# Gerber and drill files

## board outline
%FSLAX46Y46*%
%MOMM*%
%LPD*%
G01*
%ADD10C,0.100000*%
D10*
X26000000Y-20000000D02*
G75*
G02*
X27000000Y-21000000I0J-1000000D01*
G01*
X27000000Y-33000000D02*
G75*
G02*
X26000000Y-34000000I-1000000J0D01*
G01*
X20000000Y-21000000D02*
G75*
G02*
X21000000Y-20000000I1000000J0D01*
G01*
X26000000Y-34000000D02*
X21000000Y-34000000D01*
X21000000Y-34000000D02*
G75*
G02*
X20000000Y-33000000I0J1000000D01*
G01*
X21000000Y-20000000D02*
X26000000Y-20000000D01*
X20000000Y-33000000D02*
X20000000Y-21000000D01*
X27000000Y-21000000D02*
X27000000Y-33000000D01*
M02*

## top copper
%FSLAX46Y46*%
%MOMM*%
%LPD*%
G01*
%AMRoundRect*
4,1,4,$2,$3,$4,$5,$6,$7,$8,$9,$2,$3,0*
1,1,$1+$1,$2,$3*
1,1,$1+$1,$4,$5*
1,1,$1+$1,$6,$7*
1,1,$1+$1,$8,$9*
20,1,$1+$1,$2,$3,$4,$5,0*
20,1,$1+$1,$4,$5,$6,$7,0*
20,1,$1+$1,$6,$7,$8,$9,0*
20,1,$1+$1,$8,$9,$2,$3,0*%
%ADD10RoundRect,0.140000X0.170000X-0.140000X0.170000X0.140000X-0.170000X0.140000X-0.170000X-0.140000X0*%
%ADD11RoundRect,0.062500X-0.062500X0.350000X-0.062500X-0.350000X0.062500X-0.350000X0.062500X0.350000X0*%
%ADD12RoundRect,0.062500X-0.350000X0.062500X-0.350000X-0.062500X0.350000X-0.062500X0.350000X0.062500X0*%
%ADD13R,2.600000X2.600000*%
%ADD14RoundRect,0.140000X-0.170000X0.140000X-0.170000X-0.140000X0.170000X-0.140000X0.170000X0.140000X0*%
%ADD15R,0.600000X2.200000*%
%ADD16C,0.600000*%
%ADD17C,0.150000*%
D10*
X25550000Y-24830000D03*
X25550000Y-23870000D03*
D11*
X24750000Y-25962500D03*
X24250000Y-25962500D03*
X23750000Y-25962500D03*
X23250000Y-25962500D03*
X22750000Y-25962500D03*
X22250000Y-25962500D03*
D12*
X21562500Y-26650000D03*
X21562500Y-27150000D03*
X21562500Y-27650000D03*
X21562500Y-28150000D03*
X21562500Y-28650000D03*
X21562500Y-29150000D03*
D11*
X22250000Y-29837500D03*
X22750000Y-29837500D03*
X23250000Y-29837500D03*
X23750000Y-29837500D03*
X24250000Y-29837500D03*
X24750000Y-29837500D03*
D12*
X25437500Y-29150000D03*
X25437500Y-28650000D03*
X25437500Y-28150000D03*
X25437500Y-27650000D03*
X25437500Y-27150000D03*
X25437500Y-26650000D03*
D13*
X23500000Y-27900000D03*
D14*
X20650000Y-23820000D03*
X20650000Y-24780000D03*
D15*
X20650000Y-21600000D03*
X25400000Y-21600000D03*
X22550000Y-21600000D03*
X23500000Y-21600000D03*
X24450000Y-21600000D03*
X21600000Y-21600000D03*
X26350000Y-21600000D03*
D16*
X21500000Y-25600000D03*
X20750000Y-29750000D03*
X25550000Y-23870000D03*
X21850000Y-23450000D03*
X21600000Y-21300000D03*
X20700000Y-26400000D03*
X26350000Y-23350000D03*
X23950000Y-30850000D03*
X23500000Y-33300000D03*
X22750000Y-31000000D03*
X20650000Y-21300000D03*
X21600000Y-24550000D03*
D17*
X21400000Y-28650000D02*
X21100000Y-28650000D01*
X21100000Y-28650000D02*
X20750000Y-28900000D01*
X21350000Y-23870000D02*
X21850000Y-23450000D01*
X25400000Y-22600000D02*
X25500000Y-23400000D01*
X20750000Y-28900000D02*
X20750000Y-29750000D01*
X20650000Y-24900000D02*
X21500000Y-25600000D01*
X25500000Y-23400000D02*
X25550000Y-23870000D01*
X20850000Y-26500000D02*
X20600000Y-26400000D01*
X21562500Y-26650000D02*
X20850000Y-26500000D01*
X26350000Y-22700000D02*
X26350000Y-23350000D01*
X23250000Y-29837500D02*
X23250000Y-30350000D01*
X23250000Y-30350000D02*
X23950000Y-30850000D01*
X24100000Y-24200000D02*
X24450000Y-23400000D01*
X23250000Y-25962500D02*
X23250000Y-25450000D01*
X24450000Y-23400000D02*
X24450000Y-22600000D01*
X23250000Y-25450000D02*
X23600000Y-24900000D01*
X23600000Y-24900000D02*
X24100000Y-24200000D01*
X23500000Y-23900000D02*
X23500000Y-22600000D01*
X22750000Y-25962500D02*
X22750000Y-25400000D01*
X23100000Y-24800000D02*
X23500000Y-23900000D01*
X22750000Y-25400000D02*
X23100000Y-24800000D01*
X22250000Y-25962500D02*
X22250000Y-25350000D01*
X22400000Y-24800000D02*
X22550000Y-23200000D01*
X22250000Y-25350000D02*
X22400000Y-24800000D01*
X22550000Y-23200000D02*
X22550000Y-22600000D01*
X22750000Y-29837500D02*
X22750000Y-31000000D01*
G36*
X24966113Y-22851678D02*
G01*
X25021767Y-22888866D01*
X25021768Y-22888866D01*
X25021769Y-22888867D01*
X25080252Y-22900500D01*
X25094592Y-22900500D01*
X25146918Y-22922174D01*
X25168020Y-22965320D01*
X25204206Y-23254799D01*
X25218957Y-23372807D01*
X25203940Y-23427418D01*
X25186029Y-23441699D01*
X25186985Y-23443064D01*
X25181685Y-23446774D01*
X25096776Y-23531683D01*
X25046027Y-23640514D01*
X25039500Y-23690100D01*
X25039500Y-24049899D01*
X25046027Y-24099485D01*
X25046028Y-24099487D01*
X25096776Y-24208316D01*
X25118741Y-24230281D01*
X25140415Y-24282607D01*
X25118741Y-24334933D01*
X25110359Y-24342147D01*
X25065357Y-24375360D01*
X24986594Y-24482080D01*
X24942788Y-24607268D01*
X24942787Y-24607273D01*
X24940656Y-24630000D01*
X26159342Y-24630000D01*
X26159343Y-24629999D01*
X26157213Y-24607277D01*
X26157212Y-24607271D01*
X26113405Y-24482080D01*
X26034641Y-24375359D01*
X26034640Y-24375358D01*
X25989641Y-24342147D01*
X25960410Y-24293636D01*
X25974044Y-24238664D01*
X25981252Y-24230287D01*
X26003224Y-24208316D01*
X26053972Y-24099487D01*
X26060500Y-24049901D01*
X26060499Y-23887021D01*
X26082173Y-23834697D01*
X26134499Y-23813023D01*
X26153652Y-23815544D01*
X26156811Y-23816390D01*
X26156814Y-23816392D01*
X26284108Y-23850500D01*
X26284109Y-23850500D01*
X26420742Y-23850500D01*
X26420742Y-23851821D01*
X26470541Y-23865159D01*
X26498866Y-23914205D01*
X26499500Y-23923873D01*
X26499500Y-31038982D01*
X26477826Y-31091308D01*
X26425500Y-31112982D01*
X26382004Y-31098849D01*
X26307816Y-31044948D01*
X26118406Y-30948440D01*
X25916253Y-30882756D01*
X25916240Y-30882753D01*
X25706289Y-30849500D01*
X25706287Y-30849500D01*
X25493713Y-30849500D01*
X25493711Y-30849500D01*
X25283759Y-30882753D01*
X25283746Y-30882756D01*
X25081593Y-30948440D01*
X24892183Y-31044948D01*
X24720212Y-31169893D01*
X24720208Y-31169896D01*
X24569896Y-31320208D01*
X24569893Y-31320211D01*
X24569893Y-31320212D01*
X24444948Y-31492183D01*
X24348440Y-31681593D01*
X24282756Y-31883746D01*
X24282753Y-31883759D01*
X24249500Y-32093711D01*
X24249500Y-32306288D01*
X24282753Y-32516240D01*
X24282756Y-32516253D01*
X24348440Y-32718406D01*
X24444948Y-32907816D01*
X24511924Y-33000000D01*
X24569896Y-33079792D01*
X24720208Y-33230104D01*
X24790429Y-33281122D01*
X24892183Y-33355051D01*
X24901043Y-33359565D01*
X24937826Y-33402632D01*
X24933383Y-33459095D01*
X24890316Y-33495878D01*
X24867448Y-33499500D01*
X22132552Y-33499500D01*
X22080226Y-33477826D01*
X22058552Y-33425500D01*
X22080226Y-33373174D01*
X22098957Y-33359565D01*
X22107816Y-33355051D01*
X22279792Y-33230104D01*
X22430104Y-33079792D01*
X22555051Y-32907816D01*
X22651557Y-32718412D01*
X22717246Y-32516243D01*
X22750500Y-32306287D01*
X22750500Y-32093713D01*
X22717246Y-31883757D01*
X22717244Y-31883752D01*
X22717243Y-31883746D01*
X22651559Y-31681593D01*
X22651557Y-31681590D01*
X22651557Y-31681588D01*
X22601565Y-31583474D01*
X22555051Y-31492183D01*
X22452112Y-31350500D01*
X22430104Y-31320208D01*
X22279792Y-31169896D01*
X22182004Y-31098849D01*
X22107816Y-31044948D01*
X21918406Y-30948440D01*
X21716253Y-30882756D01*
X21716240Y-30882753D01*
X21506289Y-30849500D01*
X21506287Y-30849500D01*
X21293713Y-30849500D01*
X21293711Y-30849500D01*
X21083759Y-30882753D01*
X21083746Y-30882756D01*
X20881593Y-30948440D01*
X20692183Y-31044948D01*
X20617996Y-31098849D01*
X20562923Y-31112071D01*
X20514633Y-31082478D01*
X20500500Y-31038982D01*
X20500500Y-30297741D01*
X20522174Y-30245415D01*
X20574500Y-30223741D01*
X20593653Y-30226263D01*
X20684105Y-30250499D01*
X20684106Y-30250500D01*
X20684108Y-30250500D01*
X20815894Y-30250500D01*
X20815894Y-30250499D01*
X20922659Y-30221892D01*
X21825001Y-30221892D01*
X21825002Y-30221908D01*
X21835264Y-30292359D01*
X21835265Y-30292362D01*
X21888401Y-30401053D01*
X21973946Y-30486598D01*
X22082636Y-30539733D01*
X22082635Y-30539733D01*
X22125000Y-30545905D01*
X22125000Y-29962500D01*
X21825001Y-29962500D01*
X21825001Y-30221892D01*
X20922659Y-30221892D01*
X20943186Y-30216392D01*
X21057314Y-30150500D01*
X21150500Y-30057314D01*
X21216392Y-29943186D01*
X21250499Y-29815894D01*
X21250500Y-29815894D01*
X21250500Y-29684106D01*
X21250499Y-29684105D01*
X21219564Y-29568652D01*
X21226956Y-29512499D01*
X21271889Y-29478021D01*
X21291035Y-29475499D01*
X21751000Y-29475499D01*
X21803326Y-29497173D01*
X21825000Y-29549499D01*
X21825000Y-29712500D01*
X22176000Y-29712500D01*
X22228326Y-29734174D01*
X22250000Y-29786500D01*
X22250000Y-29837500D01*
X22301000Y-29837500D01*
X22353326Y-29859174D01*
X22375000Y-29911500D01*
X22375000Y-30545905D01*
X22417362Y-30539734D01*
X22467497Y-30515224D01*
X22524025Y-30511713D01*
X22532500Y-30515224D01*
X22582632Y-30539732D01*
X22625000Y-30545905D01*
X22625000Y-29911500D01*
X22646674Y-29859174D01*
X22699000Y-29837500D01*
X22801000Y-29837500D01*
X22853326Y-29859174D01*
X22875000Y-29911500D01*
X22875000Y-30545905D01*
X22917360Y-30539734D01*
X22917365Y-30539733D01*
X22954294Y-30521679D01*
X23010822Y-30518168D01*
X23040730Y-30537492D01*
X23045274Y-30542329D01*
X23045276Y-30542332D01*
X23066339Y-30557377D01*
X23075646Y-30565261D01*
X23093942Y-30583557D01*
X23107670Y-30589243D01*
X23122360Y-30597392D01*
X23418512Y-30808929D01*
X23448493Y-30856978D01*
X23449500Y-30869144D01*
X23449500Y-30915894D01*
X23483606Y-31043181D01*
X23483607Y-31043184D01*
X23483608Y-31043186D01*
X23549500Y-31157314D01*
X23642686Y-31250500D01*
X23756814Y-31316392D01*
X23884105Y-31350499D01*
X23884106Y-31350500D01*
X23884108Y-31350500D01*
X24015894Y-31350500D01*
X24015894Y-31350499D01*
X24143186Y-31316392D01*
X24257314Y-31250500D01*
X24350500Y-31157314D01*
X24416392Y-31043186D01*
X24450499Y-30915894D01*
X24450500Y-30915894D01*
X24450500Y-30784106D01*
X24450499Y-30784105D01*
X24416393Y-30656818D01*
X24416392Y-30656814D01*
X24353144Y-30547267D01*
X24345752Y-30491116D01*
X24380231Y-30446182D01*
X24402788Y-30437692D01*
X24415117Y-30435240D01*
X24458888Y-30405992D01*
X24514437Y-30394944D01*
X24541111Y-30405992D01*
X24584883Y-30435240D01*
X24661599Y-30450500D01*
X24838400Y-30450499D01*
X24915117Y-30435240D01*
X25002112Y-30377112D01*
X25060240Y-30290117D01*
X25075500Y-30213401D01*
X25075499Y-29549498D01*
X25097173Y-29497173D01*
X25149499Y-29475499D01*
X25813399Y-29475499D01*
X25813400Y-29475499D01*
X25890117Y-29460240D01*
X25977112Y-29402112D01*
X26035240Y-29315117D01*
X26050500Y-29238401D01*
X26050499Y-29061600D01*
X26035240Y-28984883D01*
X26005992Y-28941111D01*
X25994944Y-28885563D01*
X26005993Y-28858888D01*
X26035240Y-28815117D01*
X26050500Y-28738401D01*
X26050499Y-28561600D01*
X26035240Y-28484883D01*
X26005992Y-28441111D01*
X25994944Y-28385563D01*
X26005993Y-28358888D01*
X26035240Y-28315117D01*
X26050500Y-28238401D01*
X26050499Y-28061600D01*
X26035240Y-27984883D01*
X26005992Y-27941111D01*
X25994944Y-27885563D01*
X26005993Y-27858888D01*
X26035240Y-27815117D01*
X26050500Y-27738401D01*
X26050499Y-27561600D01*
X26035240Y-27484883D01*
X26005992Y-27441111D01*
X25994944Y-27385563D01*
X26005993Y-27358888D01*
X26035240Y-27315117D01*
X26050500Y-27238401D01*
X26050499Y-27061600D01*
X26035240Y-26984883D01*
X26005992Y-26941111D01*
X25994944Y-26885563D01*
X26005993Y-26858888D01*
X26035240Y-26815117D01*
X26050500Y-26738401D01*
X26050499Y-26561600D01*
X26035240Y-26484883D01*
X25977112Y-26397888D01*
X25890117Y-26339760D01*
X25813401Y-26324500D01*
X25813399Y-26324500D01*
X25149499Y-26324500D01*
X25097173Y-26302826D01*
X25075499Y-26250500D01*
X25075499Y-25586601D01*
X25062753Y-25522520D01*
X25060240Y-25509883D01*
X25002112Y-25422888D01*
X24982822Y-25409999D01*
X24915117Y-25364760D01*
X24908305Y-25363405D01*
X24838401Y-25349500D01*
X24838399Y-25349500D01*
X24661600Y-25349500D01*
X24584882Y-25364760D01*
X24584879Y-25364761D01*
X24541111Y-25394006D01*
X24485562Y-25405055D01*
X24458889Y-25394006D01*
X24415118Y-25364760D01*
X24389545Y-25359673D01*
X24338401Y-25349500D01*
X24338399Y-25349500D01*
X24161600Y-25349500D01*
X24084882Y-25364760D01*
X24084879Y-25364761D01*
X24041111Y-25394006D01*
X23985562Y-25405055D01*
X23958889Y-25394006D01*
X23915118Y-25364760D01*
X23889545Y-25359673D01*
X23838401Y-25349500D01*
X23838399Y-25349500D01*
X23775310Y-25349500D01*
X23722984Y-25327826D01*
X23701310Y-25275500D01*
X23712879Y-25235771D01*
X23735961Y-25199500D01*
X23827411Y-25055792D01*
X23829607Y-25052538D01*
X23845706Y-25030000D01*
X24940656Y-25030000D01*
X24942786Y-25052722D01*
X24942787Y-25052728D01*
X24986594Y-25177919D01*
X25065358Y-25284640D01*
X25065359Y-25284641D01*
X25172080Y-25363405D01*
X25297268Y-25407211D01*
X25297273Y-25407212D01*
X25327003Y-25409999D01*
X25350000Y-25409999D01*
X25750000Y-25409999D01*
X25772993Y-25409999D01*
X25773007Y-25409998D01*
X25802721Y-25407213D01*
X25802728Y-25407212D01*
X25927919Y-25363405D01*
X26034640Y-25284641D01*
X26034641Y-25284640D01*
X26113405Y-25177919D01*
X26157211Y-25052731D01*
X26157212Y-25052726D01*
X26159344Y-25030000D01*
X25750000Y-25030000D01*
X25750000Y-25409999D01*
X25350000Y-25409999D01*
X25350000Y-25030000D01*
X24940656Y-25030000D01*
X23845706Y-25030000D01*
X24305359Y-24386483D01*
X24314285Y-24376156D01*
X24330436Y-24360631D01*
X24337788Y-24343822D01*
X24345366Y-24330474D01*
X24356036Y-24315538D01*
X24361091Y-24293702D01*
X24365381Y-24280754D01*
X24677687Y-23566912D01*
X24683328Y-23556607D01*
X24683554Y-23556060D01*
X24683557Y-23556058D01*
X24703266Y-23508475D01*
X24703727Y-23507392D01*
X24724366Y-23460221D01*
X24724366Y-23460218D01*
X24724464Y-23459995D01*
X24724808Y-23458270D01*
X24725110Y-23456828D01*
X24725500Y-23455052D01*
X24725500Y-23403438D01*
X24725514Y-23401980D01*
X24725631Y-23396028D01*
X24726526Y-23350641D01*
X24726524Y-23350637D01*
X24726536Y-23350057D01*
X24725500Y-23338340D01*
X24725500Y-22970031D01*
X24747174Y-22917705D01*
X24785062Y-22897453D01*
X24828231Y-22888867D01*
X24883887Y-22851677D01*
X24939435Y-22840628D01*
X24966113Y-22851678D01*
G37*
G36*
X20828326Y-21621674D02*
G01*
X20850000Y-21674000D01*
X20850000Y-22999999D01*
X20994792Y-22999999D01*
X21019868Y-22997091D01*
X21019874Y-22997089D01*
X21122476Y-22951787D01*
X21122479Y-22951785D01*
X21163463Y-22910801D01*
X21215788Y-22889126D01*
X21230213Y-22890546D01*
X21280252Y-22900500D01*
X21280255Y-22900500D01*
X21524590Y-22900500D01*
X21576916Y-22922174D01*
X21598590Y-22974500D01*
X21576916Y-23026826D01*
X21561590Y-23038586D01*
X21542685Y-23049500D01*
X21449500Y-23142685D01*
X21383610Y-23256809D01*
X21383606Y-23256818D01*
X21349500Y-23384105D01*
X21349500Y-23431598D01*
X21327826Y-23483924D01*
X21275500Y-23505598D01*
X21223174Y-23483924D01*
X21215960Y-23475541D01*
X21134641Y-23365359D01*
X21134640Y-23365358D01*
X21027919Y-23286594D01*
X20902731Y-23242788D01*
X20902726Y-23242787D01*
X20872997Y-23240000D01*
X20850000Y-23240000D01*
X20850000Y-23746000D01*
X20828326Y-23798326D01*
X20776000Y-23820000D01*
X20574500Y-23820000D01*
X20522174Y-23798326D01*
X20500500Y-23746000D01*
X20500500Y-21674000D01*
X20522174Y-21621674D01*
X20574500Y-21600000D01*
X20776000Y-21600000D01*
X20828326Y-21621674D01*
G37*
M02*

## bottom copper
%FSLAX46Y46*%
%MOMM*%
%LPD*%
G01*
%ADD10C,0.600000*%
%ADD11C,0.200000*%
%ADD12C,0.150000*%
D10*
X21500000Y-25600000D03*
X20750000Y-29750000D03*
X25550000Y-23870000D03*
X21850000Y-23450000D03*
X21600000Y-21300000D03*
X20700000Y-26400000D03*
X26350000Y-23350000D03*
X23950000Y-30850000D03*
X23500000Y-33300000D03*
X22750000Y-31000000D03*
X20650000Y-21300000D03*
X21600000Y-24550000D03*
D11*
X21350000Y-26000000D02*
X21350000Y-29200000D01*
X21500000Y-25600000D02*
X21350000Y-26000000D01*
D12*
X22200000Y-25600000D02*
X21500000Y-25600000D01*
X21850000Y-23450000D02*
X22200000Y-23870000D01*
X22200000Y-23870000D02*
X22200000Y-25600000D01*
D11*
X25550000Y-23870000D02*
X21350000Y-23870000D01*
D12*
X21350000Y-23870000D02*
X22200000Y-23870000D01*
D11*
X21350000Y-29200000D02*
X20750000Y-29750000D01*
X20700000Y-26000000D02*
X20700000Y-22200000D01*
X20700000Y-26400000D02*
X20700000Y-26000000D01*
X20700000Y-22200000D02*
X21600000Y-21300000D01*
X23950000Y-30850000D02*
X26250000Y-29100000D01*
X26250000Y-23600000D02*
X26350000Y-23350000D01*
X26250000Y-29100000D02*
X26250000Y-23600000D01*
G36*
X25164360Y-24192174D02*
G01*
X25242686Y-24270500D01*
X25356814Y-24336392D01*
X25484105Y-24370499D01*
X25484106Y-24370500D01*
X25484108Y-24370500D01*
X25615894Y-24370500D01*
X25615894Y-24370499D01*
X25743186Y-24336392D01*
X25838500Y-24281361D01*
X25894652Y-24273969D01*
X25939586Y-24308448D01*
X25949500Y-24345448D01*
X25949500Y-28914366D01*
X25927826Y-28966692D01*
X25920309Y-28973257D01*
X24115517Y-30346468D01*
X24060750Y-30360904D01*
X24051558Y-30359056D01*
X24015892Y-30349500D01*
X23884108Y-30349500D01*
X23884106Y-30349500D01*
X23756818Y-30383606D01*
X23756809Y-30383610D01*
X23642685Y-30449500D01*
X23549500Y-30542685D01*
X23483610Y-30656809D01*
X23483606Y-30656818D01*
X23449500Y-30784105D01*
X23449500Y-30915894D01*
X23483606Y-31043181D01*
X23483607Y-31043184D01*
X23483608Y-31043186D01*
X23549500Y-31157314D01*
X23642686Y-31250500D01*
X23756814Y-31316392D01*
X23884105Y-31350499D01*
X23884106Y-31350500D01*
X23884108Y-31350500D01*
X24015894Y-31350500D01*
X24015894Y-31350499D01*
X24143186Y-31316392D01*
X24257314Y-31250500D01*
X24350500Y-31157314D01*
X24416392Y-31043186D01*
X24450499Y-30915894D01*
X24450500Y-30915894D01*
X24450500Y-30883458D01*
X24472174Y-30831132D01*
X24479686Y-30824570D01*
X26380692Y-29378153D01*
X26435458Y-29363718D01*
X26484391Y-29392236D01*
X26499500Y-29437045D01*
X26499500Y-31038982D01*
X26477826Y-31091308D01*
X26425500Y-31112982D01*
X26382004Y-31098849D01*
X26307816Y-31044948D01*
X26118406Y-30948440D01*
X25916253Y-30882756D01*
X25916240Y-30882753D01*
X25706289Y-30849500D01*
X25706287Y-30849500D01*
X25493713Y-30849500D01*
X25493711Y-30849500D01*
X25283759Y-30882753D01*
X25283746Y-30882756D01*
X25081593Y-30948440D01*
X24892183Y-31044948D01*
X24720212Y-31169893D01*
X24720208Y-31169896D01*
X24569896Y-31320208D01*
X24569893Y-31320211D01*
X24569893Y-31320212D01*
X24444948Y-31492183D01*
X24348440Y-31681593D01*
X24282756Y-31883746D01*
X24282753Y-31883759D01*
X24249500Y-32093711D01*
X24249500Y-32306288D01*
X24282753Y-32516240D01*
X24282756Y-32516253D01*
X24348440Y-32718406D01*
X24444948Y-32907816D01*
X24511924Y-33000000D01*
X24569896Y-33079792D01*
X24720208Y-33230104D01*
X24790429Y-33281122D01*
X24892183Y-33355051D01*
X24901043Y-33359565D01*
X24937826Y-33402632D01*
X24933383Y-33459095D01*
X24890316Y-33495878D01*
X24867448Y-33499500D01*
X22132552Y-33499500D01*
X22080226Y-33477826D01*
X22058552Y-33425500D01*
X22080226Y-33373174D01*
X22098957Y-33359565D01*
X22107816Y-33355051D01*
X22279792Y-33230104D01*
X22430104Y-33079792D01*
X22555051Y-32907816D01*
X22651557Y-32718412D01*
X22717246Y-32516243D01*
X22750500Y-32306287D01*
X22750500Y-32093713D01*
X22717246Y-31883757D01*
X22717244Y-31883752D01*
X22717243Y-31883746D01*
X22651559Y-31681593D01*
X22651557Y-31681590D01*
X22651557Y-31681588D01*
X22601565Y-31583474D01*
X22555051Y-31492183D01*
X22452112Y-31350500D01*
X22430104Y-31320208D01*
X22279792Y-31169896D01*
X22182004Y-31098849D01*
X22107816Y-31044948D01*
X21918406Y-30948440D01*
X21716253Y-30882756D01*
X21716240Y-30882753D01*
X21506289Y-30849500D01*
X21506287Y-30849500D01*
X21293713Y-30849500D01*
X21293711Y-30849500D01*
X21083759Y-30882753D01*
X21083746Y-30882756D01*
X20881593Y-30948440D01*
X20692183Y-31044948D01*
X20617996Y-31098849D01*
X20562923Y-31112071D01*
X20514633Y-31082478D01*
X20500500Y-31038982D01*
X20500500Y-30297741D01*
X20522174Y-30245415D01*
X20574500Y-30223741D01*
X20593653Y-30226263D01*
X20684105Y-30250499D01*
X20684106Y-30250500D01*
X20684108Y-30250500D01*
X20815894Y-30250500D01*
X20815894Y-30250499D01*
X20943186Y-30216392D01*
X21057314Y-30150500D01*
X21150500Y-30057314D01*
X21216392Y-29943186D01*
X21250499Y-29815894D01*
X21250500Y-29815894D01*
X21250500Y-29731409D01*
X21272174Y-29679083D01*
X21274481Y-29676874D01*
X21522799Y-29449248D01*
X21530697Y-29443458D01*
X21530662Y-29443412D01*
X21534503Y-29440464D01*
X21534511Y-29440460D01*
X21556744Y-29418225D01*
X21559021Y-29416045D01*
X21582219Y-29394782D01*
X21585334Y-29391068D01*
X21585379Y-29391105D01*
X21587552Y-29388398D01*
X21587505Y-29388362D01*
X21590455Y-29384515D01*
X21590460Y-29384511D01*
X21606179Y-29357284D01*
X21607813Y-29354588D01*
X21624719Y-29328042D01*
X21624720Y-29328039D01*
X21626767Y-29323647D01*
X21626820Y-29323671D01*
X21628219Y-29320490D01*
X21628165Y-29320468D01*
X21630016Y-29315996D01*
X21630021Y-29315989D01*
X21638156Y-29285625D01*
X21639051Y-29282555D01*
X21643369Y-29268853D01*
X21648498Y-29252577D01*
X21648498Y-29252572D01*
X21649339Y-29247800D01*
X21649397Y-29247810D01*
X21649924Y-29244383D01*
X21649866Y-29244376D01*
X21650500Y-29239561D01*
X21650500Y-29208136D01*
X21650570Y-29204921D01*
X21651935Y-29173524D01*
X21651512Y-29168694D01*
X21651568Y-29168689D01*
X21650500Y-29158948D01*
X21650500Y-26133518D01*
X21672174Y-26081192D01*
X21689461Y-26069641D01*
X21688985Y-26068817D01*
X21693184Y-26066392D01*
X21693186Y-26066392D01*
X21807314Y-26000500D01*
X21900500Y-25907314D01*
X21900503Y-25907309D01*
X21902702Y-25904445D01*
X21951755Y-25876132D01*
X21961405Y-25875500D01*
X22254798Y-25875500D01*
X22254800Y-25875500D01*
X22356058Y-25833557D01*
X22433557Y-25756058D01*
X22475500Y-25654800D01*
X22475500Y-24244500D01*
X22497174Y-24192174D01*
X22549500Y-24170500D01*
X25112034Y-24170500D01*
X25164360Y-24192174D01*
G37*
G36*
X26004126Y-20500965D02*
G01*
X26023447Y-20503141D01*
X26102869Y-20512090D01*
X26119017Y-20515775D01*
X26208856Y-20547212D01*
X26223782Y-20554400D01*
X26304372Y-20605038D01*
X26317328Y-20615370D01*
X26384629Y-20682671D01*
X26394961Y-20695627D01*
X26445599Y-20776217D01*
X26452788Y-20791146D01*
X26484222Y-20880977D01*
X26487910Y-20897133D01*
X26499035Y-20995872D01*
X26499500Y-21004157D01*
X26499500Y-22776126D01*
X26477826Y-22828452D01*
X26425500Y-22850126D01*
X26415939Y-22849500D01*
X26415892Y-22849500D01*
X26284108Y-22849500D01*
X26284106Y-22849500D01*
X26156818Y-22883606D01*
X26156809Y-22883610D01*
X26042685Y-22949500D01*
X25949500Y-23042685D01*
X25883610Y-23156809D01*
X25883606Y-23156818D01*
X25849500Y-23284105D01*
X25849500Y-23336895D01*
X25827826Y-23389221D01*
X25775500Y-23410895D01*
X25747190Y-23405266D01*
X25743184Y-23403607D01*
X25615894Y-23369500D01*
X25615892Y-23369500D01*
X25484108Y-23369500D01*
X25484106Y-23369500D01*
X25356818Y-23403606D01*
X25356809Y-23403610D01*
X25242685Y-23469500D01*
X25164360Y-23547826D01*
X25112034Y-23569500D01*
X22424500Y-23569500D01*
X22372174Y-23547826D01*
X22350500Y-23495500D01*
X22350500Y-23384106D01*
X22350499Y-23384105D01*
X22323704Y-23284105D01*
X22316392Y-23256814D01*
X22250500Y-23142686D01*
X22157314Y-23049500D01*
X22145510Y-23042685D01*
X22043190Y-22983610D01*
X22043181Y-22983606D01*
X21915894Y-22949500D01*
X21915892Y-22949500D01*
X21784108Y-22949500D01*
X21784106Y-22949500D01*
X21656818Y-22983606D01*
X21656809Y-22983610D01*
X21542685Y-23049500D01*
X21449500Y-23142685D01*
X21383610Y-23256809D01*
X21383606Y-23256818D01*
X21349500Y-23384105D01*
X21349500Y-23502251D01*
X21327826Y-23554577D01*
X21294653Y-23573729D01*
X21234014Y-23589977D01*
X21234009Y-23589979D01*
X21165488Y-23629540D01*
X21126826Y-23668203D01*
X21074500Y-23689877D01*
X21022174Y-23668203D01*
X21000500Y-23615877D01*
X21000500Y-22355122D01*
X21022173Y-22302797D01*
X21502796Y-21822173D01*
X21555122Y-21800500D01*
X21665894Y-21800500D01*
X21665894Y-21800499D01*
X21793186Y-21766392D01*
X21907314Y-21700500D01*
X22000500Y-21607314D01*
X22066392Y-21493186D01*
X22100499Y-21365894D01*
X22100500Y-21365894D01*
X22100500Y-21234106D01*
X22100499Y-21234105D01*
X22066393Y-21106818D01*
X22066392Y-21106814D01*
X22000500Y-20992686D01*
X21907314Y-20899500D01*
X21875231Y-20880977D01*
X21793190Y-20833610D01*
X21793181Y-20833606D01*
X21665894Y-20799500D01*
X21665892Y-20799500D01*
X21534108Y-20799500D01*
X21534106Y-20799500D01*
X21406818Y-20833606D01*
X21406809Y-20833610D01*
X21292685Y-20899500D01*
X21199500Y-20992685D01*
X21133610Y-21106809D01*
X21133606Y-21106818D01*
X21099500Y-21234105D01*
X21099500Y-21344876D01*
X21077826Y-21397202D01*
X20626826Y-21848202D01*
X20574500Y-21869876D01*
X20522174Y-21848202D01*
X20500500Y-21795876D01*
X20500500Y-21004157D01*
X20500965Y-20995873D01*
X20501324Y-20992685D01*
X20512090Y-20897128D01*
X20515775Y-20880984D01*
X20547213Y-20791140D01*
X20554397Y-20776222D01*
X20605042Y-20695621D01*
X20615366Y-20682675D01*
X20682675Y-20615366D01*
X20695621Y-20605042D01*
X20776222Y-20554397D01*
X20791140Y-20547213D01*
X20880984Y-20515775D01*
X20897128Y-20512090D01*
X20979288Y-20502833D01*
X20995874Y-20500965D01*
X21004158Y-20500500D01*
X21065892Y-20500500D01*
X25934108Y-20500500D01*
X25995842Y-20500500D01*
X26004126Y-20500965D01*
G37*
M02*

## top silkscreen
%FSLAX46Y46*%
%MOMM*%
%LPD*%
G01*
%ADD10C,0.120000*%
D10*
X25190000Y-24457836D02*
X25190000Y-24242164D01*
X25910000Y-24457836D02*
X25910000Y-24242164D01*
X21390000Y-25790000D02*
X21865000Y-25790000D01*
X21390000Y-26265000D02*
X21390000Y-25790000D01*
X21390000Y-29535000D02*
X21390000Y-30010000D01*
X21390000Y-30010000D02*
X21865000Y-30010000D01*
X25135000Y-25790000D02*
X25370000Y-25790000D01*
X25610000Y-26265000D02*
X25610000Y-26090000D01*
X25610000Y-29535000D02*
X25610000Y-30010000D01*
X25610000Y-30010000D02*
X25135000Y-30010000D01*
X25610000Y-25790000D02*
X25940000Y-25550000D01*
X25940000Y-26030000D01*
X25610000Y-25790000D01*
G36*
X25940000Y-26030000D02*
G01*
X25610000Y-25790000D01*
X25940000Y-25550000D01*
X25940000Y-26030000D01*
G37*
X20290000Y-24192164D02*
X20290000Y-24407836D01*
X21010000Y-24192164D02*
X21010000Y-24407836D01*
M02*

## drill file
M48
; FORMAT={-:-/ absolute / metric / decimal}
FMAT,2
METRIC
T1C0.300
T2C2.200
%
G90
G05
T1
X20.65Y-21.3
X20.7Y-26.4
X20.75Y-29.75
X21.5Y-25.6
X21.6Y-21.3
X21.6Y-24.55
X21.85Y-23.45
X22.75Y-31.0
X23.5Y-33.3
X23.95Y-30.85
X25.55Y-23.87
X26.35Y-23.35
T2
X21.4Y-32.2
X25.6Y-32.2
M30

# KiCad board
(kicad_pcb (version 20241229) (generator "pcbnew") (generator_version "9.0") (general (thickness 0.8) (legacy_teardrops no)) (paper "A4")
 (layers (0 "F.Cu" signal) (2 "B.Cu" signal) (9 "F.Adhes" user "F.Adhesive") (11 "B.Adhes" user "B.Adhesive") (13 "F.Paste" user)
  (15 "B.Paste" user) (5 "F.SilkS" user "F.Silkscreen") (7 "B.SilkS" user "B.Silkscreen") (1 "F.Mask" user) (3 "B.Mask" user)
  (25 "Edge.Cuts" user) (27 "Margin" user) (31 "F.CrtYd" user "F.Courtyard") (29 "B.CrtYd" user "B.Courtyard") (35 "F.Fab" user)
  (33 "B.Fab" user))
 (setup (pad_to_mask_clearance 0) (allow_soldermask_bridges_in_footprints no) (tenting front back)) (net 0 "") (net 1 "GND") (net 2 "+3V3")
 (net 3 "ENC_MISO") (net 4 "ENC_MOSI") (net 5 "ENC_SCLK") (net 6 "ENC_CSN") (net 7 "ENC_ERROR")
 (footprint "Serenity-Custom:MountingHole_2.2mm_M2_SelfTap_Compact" (layer "F.Cu") (at 21.4 32.2)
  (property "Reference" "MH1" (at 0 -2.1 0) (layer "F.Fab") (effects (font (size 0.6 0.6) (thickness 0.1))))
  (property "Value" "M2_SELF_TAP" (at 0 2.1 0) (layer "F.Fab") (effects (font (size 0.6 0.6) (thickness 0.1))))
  (pad "" np_thru_hole circle (at 0 0) (size 2.2 2.2) (drill 2.2) (layers "*.Cu" "*.Mask")))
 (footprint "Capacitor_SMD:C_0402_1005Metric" (layer "F.Cu") (at 25.55 24.35 90)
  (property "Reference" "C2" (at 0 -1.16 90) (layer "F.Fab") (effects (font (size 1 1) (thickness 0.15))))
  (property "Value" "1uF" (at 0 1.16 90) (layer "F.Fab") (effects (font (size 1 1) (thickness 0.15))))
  (fp_line (start -0.107836 -0.36) (end 0.107836 -0.36) (stroke (width 0.12) (type solid)) (layer "F.SilkS"))
  (fp_line (start -0.107836 0.36) (end 0.107836 0.36) (stroke (width 0.12) (type solid)) (layer "F.SilkS"))
  (pad "1" smd roundrect (at -0.48 0 90) (size 0.56 0.62) (layers "F.Cu" "F.Mask" "F.Paste") (roundrect_rratio 0.25) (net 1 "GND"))
  (pad "2" smd roundrect (at 0.48 0 90) (size 0.56 0.62) (layers "F.Cu" "F.Mask" "F.Paste") (roundrect_rratio 0.25) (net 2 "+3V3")))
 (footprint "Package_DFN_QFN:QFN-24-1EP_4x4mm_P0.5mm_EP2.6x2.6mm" (layer "F.Cu") (at 23.5 27.9 -90)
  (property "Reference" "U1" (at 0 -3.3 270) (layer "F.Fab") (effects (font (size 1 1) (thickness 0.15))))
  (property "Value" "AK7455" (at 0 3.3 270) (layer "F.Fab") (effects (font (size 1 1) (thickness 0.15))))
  (fp_line (start -2.11 2.11) (end -2.11 1.635) (stroke (width 0.12) (type solid)) (layer "F.SilkS"))
  (fp_line (start -1.635 2.11) (end -2.11 2.11) (stroke (width 0.12) (type solid)) (layer "F.SilkS"))
  (fp_line (start 1.635 2.11) (end 2.11 2.11) (stroke (width 0.12) (type solid)) (layer "F.SilkS"))
  (fp_line (start 2.11 2.11) (end 2.11 1.635) (stroke (width 0.12) (type solid)) (layer "F.SilkS"))
  (fp_line (start -2.11 -1.635) (end -2.11 -1.87) (stroke (width 0.12) (type solid)) (layer "F.SilkS"))
  (fp_line (start -1.635 -2.11) (end -1.81 -2.11) (stroke (width 0.12) (type solid)) (layer "F.SilkS"))
  (fp_line (start 1.635 -2.11) (end 2.11 -2.11) (stroke (width 0.12) (type solid)) (layer "F.SilkS"))
  (fp_line (start 2.11 -2.11) (end 2.11 -1.635) (stroke (width 0.12) (type solid)) (layer "F.SilkS"))
  (fp_poly (pts (xy -2.11 -2.11) (xy -2.35 -2.44) (xy -1.87 -2.44)) (stroke (width 0.12) (type solid)) (fill yes) (layer "F.SilkS"))
  (pad "" smd roundrect (at -0.65 -0.65 270) (size 1.05 1.05) (layers "F.Paste") (roundrect_rratio 0.238095))
  (pad "" smd roundrect (at -0.65 0.65 270) (size 1.05 1.05) (layers "F.Paste") (roundrect_rratio 0.238095))
  (pad "" smd roundrect (at 0.65 -0.65 270) (size 1.05 1.05) (layers "F.Paste") (roundrect_rratio 0.238095))
  (pad "" smd roundrect (at 0.65 0.65 270) (size 1.05 1.05) (layers "F.Paste") (roundrect_rratio 0.238095))
  (pad "1" smd roundrect (at -1.9375 -1.25 270) (size 0.825 0.25) (layers "F.Cu" "F.Mask" "F.Paste") (roundrect_rratio 0.25))
  (pad "2" smd roundrect (at -1.9375 -0.75 270) (size 0.825 0.25) (layers "F.Cu" "F.Mask" "F.Paste") (roundrect_rratio 0.25))
  (pad "3" smd roundrect (at -1.9375 -0.25 270) (size 0.825 0.25) (layers "F.Cu" "F.Mask" "F.Paste") (roundrect_rratio 0.25))
  (pad "4" smd roundrect (at -1.9375 0.25 270) (size 0.825 0.25) (layers "F.Cu" "F.Mask" "F.Paste") (roundrect_rratio 0.25)
   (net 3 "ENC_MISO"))
  (pad "5" smd roundrect (at -1.9375 0.75 270) (size 0.825 0.25) (layers "F.Cu" "F.Mask" "F.Paste") (roundrect_rratio 0.25)
   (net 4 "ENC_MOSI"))
  (pad "6" smd roundrect (at -1.9375 1.25 270) (size 0.825 0.25) (layers "F.Cu" "F.Mask" "F.Paste") (roundrect_rratio 0.25)
   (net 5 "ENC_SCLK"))
  (pad "7" smd roundrect (at -1.25 1.9375 270) (size 0.25 0.825) (layers "F.Cu" "F.Mask" "F.Paste") (roundrect_rratio 0.25)
   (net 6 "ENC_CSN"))
  (pad "8" smd roundrect (at -0.75 1.9375 270) (size 0.25 0.825) (layers "F.Cu" "F.Mask" "F.Paste") (roundrect_rratio 0.25))
  (pad "9" smd roundrect (at -0.25 1.9375 270) (size 0.25 0.825) (layers "F.Cu" "F.Mask" "F.Paste") (roundrect_rratio 0.25))
  (pad "10" smd roundrect (at 0.25 1.9375 270) (size 0.25 0.825) (layers "F.Cu" "F.Mask" "F.Paste") (roundrect_rratio 0.25))
  (pad "11" smd roundrect (at 0.75 1.9375 270) (size 0.25 0.825) (layers "F.Cu" "F.Mask" "F.Paste") (roundrect_rratio 0.25) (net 2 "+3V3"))
  (pad "12" smd roundrect (at 1.25 1.9375 270) (size 0.25 0.825) (layers "F.Cu" "F.Mask" "F.Paste") (roundrect_rratio 0.25))
  (pad "13" smd roundrect (at 1.9375 1.25 270) (size 0.825 0.25) (layers "F.Cu" "F.Mask" "F.Paste") (roundrect_rratio 0.25) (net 1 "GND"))
  (pad "14" smd roundrect (at 1.9375 0.75 270) (size 0.825 0.25) (layers "F.Cu" "F.Mask" "F.Paste") (roundrect_rratio 0.25) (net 1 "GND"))
  (pad "15" smd roundrect (at 1.9375 0.25 270) (size 0.825 0.25) (layers "F.Cu" "F.Mask" "F.Paste") (roundrect_rratio 0.25)
   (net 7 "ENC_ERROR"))
  (pad "16" smd roundrect (at 1.9375 -0.25 270) (size 0.825 0.25) (layers "F.Cu" "F.Mask" "F.Paste") (roundrect_rratio 0.25))
  (pad "17" smd roundrect (at 1.9375 -0.75 270) (size 0.825 0.25) (layers "F.Cu" "F.Mask" "F.Paste") (roundrect_rratio 0.25))
  (pad "18" smd roundrect (at 1.9375 -1.25 270) (size 0.825 0.25) (layers "F.Cu" "F.Mask" "F.Paste") (roundrect_rratio 0.25))
  (pad "19" smd roundrect (at 1.25 -1.9375 270) (size 0.25 0.825) (layers "F.Cu" "F.Mask" "F.Paste") (roundrect_rratio 0.25))
  (pad "20" smd roundrect (at 0.75 -1.9375 270) (size 0.25 0.825) (layers "F.Cu" "F.Mask" "F.Paste") (roundrect_rratio 0.25))
  (pad "21" smd roundrect (at 0.25 -1.9375 270) (size 0.25 0.825) (layers "F.Cu" "F.Mask" "F.Paste") (roundrect_rratio 0.25))
  (pad "22" smd roundrect (at -0.25 -1.9375 270) (size 0.25 0.825) (layers "F.Cu" "F.Mask" "F.Paste") (roundrect_rratio 0.25))
  (pad "23" smd roundrect (at -0.75 -1.9375 270) (size 0.25 0.825) (layers "F.Cu" "F.Mask" "F.Paste") (roundrect_rratio 0.25))
  (pad "24" smd roundrect (at -1.25 -1.9375 270) (size 0.25 0.825) (layers "F.Cu" "F.Mask" "F.Paste") (roundrect_rratio 0.25))
  (pad "25" smd rect (at 0 0 270) (size 2.6 2.6) (layers "F.Cu" "F.Mask") (zone_connect 2)))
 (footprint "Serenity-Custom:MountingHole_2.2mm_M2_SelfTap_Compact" (layer "F.Cu") (at 25.6 32.2)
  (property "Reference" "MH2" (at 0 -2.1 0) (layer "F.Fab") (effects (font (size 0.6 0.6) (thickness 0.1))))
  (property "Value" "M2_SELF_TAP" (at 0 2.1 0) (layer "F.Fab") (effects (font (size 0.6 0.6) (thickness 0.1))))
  (pad "" np_thru_hole circle (at 0 0) (size 2.2 2.2) (drill 2.2) (layers "*.Cu" "*.Mask")))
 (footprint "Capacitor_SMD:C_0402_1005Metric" (layer "F.Cu") (at 20.65 24.3 -90)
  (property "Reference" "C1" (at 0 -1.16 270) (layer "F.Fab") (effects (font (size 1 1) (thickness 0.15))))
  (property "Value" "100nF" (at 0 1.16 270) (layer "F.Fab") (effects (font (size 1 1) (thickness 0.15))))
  (fp_line (start -0.107836 0.36) (end 0.107836 0.36) (stroke (width 0.12) (type solid)) (layer "F.SilkS"))
  (fp_line (start -0.107836 -0.36) (end 0.107836 -0.36) (stroke (width 0.12) (type solid)) (layer "F.SilkS"))
  (pad "1" smd roundrect (at -0.48 0 270) (size 0.56 0.62) (layers "F.Cu" "F.Mask" "F.Paste") (roundrect_rratio 0.25) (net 1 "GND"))
  (pad "2" smd roundrect (at 0.48 0 270) (size 0.56 0.62) (layers "F.Cu" "F.Mask" "F.Paste") (roundrect_rratio 0.25) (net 2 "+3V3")))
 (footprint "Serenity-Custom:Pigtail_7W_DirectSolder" (layer "F.Cu") (at 23.5 21.6)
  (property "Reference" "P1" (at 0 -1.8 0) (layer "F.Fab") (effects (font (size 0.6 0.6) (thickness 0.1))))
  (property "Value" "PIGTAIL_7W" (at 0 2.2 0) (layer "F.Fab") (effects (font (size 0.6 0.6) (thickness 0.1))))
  (pad "1" smd rect (at -2.85 0) (size 0.6 2.2) (layers "F.Cu" "F.Mask" "F.Paste") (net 1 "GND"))
  (pad "2" smd rect (at 1.9 0) (size 0.6 2.2) (layers "F.Cu" "F.Mask" "F.Paste") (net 2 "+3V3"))
  (pad "3" smd rect (at -0.95 0) (size 0.6 2.2) (layers "F.Cu" "F.Mask" "F.Paste") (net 5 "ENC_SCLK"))
  (pad "4" smd rect (at 0 0) (size 0.6 2.2) (layers "F.Cu" "F.Mask" "F.Paste") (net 4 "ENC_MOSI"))
  (pad "5" smd rect (at 0.95 0) (size 0.6 2.2) (layers "F.Cu" "F.Mask" "F.Paste") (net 3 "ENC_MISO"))
  (pad "6" smd rect (at -1.9 0) (size 0.6 2.2) (layers "F.Cu" "F.Mask" "F.Paste") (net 6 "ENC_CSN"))
  (pad "7" smd rect (at 2.85 0) (size 0.6 2.2) (layers "F.Cu" "F.Mask" "F.Paste") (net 7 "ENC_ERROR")))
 (gr_arc (start 26 20) (mid 26.707107 20.292893) (end 27 21) (stroke (width 0.1) (type solid)) (layer "Edge.Cuts"))
 (gr_arc (start 27 33) (mid 26.707107 33.707107) (end 26 34) (stroke (width 0.1) (type solid)) (layer "Edge.Cuts"))
 (gr_arc (start 20 21) (mid 20.292893 20.292893) (end 21 20) (stroke (width 0.1) (type solid)) (layer "Edge.Cuts"))
 (gr_line (start 26 34) (end 21 34) (stroke (width 0.1) (type solid)) (layer "Edge.Cuts"))
 (gr_arc (start 21 34) (mid 20.292893 33.707107) (end 20 33) (stroke (width 0.1) (type solid)) (layer "Edge.Cuts"))
 (gr_line (start 21 20) (end 26 20) (stroke (width 0.1) (type solid)) (layer "Edge.Cuts"))
 (gr_line (start 20 33) (end 20 21) (stroke (width 0.1) (type solid)) (layer "Edge.Cuts"))
 (gr_line (start 27 21) (end 27 33) (stroke (width 0.1) (type solid)) (layer "Edge.Cuts"))
 (segment (start 21.4 28.65) (end 21.1 28.65) (width 0.15) (layer "F.Cu") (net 2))
 (segment (start 21.1 28.65) (end 20.75 28.9) (width 0.15) (layer "F.Cu") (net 2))
 (segment (start 21.35 23.87) (end 21.85 23.45) (width 0.15) (layer "F.Cu") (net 2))
 (segment (start 25.4 22.6) (end 25.5 23.4) (width 0.15) (layer "F.Cu") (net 2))
 (segment (start 20.75 28.9) (end 20.75 29.75) (width 0.15) (layer "F.Cu") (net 2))
 (segment (start 20.65 24.9) (end 21.5 25.6) (width 0.15) (layer "F.Cu") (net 2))
 (segment (start 25.5 23.4) (end 25.55 23.87) (width 0.15) (layer "F.Cu") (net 2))
 (via (at 21.5 25.6) (size 0.6) (drill 0.3) (layers "F.Cu" "B.Cu") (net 2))
 (via (at 20.75 29.75) (size 0.6) (drill 0.3) (layers "F.Cu" "B.Cu") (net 2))
 (via (at 25.55 23.87) (size 0.6) (drill 0.3) (layers "F.Cu" "B.Cu") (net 2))
 (via (at 21.85 23.45) (size 0.6) (drill 0.3) (layers "F.Cu" "B.Cu") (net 2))
 (segment (start 21.35 26) (end 21.35 29.2) (width 0.2) (layer "B.Cu") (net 2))
 (segment (start 21.5 25.6) (end 21.35 26) (width 0.2) (layer "B.Cu") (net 2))
 (segment (start 22.2 25.6) (end 21.5 25.6) (width 0.15) (layer "B.Cu") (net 2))
 (segment (start 21.85 23.45) (end 22.2 23.87) (width 0.15) (layer "B.Cu") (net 2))
 (segment (start 22.2 23.87) (end 22.2 25.6) (width 0.15) (layer "B.Cu") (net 2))
 (segment (start 25.55 23.87) (end 21.35 23.87) (width 0.2) (layer "B.Cu") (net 2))
 (segment (start 21.35 23.87) (end 22.2 23.87) (width 0.15) (layer "B.Cu") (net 2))
 (segment (start 21.35 29.2) (end 20.75 29.75) (width 0.2) (layer "B.Cu") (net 2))
 (segment (start 20.85 26.5) (end 20.6 26.4) (width 0.15) (layer "F.Cu") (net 6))
 (segment (start 21.5625 26.65) (end 20.85 26.5) (width 0.15) (layer "F.Cu") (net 6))
 (via (at 21.6 21.3) (size 0.6) (drill 0.3) (layers "F.Cu" "B.Cu") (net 6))
 (via (at 20.7 26.4) (size 0.6) (drill 0.3) (layers "F.Cu" "B.Cu") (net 6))
 (segment (start 20.7 26) (end 20.7 22.2) (width 0.2) (layer "B.Cu") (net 6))
 (segment (start 20.7 26.4) (end 20.7 26) (width 0.2) (layer "B.Cu") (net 6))
 (segment (start 20.7 22.2) (end 21.6 21.3) (width 0.2) (layer "B.Cu") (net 6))
 (segment (start 26.35 22.7) (end 26.35 23.35) (width 0.15) (layer "F.Cu") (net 7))
 (segment (start 23.25 29.8375) (end 23.25 30.35) (width 0.15) (layer "F.Cu") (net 7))
 (segment (start 23.25 30.35) (end 23.95 30.85) (width 0.15) (layer "F.Cu") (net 7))
 (via (at 26.35 23.35) (size 0.6) (drill 0.3) (layers "F.Cu" "B.Cu") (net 7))
 (via (at 23.95 30.85) (size 0.6) (drill 0.3) (layers "F.Cu" "B.Cu") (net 7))
 (segment (start 23.95 30.85) (end 26.25 29.1) (width 0.2) (layer "B.Cu") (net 7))
 (segment (start 26.25 23.6) (end 26.35 23.35) (width 0.2) (layer "B.Cu") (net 7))
 (segment (start 26.25 29.1) (end 26.25 23.6) (width 0.2) (layer "B.Cu") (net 7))
 (segment (start 24.1 24.2) (end 24.45 23.4) (width 0.15) (layer "F.Cu") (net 3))
 (segment (start 23.25 25.9625) (end 23.25 25.45) (width 0.15) (layer "F.Cu") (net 3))
 (segment (start 24.45 23.4) (end 24.45 22.6) (width 0.15) (layer "F.Cu") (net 3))
 (segment (start 23.25 25.45) (end 23.6 24.9) (width 0.15) (layer "F.Cu") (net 3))
 (segment (start 23.6 24.9) (end 24.1 24.2) (width 0.15) (layer "F.Cu") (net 3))
 (segment (start 23.5 23.9) (end 23.5 22.6) (width 0.15) (layer "F.Cu") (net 4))
 (segment (start 22.75 25.9625) (end 22.75 25.4) (width 0.15) (layer "F.Cu") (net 4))
 (segment (start 23.1 24.8) (end 23.5 23.9) (width 0.15) (layer "F.Cu") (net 4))
 (segment (start 22.75 25.4) (end 23.1 24.8) (width 0.15) (layer "F.Cu") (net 4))
 (segment (start 22.25 25.9625) (end 22.25 25.35) (width 0.15) (layer "F.Cu") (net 5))
 (segment (start 22.4 24.8) (end 22.55 23.2) (width 0.15) (layer "F.Cu") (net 5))
 (segment (start 22.25 25.35) (end 22.4 24.8) (width 0.15) (layer "F.Cu") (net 5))
 (segment (start 22.55 23.2) (end 22.55 22.6) (width 0.15) (layer "F.Cu") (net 5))
 (segment (start 22.75 29.8375) (end 22.75 31) (width 0.15) (layer "F.Cu") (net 1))
 (via (at 23.5 33.3) (size 0.6) (drill 0.3) (layers "F.Cu" "B.Cu") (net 1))
 (via (at 22.75 31) (size 0.6) (drill 0.3) (layers "F.Cu" "B.Cu") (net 1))
 (via (at 20.65 21.3) (size 0.6) (drill 0.3) (layers "F.Cu" "B.Cu") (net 1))
 (via (at 21.6 24.55) (size 0.6) (drill 0.3) (layers "F.Cu" "B.Cu") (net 1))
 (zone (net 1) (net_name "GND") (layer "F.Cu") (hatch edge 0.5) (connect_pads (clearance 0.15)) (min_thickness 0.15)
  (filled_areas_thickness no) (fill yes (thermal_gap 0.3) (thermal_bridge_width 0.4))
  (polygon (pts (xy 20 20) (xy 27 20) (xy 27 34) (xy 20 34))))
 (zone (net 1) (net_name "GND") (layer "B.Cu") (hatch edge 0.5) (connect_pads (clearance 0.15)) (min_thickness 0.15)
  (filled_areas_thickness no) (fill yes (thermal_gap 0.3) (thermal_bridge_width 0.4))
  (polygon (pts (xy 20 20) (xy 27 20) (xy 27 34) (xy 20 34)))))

